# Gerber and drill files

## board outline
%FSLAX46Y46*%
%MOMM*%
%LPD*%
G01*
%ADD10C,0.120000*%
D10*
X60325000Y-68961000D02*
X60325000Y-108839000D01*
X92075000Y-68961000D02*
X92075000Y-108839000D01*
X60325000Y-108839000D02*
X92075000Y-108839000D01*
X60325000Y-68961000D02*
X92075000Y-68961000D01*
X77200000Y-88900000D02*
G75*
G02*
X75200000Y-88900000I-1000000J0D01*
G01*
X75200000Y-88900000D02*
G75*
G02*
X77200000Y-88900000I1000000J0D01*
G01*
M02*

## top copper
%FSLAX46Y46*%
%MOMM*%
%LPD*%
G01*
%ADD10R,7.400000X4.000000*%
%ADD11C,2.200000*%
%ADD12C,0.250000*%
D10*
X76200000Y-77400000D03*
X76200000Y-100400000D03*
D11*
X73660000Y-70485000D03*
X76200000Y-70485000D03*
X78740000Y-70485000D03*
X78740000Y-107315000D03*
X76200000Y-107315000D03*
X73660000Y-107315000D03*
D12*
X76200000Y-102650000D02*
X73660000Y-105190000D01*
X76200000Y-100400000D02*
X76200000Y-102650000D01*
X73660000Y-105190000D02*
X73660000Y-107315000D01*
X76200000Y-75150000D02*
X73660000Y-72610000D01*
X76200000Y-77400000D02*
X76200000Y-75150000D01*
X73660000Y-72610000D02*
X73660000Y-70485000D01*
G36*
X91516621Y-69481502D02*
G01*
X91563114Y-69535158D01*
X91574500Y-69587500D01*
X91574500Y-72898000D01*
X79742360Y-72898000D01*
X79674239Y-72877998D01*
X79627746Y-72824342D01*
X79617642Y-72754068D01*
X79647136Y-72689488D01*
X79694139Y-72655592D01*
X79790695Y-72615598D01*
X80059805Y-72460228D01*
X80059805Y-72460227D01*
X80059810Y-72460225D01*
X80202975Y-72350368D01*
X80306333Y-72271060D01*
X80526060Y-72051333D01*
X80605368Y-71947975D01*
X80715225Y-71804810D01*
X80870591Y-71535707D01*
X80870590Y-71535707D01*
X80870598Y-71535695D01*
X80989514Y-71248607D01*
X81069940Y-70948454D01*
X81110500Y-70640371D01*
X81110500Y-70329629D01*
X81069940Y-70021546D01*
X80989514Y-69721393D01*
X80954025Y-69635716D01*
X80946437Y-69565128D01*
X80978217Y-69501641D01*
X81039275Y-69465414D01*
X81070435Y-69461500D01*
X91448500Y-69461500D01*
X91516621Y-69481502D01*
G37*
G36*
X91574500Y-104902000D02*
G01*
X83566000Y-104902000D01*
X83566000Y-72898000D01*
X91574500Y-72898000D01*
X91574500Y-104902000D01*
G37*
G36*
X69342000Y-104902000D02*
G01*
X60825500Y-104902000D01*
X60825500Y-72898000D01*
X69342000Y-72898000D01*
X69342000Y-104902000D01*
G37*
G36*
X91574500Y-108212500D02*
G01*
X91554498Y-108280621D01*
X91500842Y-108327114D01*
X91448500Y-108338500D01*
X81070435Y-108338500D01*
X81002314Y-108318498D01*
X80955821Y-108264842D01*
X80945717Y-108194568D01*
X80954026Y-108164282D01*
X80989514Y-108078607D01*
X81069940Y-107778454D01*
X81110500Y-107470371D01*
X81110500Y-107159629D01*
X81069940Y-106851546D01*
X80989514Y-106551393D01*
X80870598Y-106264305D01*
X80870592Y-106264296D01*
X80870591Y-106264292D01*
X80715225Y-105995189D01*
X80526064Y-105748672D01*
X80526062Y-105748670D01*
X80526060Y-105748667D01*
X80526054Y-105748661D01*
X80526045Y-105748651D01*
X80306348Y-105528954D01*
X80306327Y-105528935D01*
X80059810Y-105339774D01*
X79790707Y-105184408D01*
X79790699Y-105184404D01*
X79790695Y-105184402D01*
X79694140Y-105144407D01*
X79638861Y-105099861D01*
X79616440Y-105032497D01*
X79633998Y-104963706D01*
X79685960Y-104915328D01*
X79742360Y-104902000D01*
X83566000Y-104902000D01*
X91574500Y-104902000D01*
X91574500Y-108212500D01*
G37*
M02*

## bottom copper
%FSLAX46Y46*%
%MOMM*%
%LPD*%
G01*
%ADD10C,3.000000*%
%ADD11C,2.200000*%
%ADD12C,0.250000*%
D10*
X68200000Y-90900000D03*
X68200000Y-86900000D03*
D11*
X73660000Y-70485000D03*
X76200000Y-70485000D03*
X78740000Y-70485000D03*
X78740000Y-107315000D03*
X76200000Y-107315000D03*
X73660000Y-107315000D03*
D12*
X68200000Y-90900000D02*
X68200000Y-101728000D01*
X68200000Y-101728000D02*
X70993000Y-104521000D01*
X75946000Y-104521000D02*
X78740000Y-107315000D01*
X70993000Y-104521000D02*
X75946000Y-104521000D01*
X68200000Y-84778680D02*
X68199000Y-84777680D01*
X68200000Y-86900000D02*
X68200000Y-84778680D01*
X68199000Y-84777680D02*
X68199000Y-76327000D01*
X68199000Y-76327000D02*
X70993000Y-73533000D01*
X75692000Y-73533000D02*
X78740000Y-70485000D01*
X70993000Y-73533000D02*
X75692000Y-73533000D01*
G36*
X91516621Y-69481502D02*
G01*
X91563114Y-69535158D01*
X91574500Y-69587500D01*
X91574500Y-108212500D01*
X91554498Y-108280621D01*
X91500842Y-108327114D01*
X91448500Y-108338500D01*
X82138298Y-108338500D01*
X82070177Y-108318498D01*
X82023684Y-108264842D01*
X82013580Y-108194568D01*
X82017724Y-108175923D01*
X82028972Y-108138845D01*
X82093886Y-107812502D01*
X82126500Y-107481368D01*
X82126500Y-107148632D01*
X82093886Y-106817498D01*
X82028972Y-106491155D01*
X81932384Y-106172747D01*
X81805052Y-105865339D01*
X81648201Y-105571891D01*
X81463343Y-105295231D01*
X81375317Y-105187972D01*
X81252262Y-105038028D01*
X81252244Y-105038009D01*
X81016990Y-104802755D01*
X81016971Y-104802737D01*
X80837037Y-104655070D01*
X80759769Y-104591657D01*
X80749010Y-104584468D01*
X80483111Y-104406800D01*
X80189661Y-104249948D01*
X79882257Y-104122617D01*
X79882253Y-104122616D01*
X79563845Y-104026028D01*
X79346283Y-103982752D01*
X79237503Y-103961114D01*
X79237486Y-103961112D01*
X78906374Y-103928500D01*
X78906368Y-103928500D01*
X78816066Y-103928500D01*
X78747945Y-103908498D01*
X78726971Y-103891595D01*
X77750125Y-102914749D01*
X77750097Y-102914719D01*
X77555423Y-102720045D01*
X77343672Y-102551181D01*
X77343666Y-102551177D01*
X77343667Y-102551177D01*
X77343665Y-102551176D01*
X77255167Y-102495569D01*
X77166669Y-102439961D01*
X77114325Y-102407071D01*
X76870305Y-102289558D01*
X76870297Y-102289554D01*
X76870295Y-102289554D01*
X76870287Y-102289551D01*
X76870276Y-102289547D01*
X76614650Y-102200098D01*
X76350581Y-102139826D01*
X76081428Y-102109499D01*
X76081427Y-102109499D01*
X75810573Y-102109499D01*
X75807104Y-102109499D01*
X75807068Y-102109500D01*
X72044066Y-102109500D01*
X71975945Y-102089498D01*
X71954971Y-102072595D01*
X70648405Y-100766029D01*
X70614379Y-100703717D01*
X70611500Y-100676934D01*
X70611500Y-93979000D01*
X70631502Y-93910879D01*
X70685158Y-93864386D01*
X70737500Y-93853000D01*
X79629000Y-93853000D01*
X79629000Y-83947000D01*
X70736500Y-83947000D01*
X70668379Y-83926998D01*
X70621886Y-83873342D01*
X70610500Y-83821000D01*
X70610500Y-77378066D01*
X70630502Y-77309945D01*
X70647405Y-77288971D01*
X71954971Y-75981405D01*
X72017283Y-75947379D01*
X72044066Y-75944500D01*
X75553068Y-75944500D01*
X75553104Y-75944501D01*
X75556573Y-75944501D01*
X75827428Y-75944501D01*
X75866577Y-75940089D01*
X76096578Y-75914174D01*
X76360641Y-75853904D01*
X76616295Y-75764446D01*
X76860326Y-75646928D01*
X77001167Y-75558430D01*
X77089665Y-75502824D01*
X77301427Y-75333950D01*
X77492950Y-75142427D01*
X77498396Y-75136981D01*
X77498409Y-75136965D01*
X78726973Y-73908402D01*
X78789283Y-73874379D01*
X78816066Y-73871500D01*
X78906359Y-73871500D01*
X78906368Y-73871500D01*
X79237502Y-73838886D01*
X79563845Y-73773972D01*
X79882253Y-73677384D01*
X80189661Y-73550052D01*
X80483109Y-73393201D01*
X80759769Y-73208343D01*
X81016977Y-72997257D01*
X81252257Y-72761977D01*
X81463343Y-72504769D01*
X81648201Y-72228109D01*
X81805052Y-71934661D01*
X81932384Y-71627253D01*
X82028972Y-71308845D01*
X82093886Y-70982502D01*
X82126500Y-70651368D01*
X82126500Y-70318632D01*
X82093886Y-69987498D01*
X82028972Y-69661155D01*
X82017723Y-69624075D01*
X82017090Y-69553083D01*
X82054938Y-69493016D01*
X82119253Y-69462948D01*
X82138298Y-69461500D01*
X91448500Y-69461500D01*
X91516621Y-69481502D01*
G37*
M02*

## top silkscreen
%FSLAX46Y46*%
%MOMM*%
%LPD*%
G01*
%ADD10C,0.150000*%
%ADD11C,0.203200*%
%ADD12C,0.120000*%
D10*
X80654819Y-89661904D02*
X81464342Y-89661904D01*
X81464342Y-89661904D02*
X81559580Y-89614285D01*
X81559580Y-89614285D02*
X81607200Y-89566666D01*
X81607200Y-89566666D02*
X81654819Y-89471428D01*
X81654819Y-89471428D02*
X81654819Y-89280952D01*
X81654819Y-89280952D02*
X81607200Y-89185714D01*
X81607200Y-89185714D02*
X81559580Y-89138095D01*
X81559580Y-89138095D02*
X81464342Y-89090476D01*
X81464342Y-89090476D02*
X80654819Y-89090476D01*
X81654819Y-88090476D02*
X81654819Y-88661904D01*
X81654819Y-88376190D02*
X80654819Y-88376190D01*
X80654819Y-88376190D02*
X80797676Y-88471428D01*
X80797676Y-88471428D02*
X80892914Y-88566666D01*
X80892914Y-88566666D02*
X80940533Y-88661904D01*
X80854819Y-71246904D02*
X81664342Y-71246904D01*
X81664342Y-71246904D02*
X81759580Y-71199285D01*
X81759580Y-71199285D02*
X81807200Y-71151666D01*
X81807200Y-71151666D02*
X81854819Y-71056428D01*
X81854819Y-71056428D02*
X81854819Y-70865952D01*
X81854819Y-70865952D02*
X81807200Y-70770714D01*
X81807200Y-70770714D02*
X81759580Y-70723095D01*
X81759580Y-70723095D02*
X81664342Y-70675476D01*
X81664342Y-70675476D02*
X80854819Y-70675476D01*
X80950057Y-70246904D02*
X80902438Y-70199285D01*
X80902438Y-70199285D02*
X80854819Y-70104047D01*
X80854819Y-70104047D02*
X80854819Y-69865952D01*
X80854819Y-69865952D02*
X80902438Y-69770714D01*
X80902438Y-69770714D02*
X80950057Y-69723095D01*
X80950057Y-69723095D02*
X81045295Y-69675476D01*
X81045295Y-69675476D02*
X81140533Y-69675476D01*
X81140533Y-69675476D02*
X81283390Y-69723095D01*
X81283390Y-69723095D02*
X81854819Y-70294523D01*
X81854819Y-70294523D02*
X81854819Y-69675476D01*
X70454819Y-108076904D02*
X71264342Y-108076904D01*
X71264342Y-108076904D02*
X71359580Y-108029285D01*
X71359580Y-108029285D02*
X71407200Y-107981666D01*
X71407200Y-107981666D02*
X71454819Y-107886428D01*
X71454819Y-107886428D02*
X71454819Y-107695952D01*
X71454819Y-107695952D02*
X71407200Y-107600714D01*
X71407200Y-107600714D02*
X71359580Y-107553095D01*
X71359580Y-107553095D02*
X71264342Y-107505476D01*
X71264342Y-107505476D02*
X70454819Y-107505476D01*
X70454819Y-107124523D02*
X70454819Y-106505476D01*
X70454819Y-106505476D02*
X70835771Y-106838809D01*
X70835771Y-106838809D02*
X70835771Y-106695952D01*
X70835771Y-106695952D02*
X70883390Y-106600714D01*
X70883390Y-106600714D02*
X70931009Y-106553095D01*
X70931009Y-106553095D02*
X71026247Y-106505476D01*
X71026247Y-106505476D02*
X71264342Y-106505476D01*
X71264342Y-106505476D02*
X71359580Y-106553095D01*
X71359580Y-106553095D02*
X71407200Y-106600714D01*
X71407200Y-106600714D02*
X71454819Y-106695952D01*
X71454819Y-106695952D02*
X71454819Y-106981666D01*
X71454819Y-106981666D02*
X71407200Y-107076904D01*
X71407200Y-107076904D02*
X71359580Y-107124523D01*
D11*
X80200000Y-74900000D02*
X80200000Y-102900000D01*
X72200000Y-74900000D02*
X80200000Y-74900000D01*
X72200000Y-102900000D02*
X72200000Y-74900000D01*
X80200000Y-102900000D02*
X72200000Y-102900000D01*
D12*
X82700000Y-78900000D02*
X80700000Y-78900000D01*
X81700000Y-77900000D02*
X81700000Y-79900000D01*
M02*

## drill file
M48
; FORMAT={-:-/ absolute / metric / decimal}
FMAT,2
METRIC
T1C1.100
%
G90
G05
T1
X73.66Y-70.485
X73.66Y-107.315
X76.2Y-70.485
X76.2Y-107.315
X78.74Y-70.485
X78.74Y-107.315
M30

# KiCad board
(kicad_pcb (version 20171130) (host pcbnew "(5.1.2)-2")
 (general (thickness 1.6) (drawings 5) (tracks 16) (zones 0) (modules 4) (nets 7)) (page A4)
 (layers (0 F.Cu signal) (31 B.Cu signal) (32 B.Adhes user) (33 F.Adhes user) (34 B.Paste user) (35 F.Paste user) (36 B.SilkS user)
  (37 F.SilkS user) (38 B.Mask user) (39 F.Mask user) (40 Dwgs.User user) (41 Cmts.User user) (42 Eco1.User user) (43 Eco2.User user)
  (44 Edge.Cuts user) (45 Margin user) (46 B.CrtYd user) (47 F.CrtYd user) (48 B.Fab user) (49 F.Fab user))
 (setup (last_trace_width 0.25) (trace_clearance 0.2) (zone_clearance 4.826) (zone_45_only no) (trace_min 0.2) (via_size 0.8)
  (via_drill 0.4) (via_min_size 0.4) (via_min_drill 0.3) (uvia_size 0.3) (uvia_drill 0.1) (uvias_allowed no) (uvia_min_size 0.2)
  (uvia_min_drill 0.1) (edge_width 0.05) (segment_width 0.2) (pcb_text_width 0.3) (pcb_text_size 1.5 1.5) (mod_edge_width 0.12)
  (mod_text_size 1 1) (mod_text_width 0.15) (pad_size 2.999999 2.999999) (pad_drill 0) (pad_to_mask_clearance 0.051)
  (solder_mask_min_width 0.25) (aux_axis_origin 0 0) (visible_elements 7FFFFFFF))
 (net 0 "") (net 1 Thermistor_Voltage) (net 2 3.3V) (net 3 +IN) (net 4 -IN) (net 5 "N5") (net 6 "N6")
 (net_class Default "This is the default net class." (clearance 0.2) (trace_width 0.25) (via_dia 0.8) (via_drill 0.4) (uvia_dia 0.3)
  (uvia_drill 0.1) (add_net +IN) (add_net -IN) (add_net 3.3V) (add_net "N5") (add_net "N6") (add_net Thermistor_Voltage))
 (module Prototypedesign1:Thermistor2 (layer B.Cu) (at 76.2 88.9 180)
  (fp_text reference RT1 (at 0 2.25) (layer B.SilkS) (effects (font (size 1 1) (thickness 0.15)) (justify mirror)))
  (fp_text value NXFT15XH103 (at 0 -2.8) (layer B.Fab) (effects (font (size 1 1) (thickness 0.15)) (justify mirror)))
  (pad 2 smd circle (at 8 -2 180) (size 3 3) (layers B.Cu B.Paste B.Mask) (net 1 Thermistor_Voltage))
  (pad 1 smd circle (at 8 2 180) (size 3 3) (layers B.Cu B.Paste B.Mask) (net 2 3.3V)))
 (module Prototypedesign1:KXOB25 (layer F.Cu) (at 76.2 88.9 270)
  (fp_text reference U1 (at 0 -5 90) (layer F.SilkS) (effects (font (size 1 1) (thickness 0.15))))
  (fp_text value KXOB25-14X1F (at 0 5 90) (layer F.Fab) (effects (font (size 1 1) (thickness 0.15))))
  (fp_line (start -14 -4) (end 14 -4) (layer F.SilkS) (width 0.2032))
  (fp_line (start -14 4) (end -14 -4) (layer F.SilkS) (width 0.2032))
  (fp_line (start 14 4) (end -14 4) (layer F.SilkS) (width 0.2032))
  (fp_line (start 14 -4) (end 14 4) (layer F.SilkS) (width 0.2032))
  (fp_line (start -10 -6.5) (end -10 -4.5) (layer F.SilkS) (width 0.12))
  (fp_line (start -11 -5.5) (end -9 -5.5) (layer F.SilkS) (width 0.12))
  (pad 1 smd rect (at -11.5 0 270) (size 4 7.4) (layers F.Cu F.Paste F.Mask) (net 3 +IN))
  (pad 2 smd rect (at 11.5 0 270) (size 4 7.4) (layers F.Cu F.Paste F.Mask) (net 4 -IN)))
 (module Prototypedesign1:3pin (layer F.Cu) (at 76.2 70.485 270)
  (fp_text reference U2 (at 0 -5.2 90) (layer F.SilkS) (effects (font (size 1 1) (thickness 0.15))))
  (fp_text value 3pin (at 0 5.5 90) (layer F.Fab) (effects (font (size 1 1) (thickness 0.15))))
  (pad 3 thru_hole circle (at 0 2.54 270) (size 2.2 2.2) (drill 1.1) (layers *.Cu *.Mask) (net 3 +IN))
  (pad 2 thru_hole circle (at 0 0 270) (size 2.2 2.2) (drill 1.1) (layers *.Cu *.Mask) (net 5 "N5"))
  (pad 1 thru_hole circle (at 0 -2.54 270) (size 2.2 2.2) (drill 1.1) (layers *.Cu *.Mask) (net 2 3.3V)))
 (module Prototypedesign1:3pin (layer F.Cu) (at 76.2 107.315 90)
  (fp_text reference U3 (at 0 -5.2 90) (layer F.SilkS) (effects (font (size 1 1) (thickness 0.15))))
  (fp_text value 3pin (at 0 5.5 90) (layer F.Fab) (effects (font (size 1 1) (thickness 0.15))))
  (pad 3 thru_hole circle (at 0 2.54 90) (size 2.2 2.2) (drill 1.1) (layers *.Cu *.Mask) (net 1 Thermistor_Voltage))
  (pad 2 thru_hole circle (at 0 0 90) (size 2.2 2.2) (drill 1.1) (layers *.Cu *.Mask) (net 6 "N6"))
  (pad 1 thru_hole circle (at 0 -2.54 90) (size 2.2 2.2) (drill 1.1) (layers *.Cu *.Mask) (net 4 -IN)))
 (gr_line (start 60.325 68.961) (end 60.325 108.839) (layer Edge.Cuts) (width 0.12))
 (gr_line (start 92.075 68.961) (end 92.075 108.839) (layer Edge.Cuts) (width 0.12))
 (gr_line (start 60.325 108.839) (end 92.075 108.839) (layer Edge.Cuts) (width 0.12))
 (gr_line (start 60.325 68.961) (end 92.075 68.961) (layer Edge.Cuts) (width 0.12))
 (gr_circle (center 76.2 88.9) (end 77.2 88.9) (layer Edge.Cuts) (width 0.12))
 (segment (start 68.2 90.9) (end 68.2 101.728) (width 0.25) (layer B.Cu) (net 1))
 (segment (start 68.2 101.728) (end 70.993 104.521) (width 0.25) (layer B.Cu) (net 1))
 (segment (start 75.946 104.521) (end 78.74 107.315) (width 0.25) (layer B.Cu) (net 1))
 (segment (start 70.993 104.521) (end 75.946 104.521) (width 0.25) (layer B.Cu) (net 1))
 (segment (start 68.2 84.77868) (end 68.199 84.77768) (width 0.25) (layer B.Cu) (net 2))
 (segment (start 68.2 86.9) (end 68.2 84.77868) (width 0.25) (layer B.Cu) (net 2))
 (segment (start 68.199 84.77768) (end 68.199 76.327) (width 0.25) (layer B.Cu) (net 2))
 (segment (start 68.199 76.327) (end 70.993 73.533) (width 0.25) (layer B.Cu) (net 2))
 (segment (start 75.692 73.533) (end 78.74 70.485) (width 0.25) (layer B.Cu) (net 2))
 (segment (start 70.993 73.533) (end 75.692 73.533) (width 0.25) (layer B.Cu) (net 2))
 (segment (start 76.2 102.65) (end 73.66 105.19) (width 0.25) (layer F.Cu) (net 4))
 (segment (start 76.2 100.4) (end 76.2 102.65) (width 0.25) (layer F.Cu) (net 4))
 (segment (start 73.66 105.19) (end 73.66 107.315) (width 0.25) (layer F.Cu) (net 4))
 (segment (start 76.2 75.15) (end 73.66 72.61) (width 0.25) (layer F.Cu) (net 3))
 (segment (start 76.2 77.4) (end 76.2 75.15) (width 0.25) (layer F.Cu) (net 3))
 (segment (start 73.66 72.61) (end 73.66 70.485) (width 0.25) (layer F.Cu) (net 3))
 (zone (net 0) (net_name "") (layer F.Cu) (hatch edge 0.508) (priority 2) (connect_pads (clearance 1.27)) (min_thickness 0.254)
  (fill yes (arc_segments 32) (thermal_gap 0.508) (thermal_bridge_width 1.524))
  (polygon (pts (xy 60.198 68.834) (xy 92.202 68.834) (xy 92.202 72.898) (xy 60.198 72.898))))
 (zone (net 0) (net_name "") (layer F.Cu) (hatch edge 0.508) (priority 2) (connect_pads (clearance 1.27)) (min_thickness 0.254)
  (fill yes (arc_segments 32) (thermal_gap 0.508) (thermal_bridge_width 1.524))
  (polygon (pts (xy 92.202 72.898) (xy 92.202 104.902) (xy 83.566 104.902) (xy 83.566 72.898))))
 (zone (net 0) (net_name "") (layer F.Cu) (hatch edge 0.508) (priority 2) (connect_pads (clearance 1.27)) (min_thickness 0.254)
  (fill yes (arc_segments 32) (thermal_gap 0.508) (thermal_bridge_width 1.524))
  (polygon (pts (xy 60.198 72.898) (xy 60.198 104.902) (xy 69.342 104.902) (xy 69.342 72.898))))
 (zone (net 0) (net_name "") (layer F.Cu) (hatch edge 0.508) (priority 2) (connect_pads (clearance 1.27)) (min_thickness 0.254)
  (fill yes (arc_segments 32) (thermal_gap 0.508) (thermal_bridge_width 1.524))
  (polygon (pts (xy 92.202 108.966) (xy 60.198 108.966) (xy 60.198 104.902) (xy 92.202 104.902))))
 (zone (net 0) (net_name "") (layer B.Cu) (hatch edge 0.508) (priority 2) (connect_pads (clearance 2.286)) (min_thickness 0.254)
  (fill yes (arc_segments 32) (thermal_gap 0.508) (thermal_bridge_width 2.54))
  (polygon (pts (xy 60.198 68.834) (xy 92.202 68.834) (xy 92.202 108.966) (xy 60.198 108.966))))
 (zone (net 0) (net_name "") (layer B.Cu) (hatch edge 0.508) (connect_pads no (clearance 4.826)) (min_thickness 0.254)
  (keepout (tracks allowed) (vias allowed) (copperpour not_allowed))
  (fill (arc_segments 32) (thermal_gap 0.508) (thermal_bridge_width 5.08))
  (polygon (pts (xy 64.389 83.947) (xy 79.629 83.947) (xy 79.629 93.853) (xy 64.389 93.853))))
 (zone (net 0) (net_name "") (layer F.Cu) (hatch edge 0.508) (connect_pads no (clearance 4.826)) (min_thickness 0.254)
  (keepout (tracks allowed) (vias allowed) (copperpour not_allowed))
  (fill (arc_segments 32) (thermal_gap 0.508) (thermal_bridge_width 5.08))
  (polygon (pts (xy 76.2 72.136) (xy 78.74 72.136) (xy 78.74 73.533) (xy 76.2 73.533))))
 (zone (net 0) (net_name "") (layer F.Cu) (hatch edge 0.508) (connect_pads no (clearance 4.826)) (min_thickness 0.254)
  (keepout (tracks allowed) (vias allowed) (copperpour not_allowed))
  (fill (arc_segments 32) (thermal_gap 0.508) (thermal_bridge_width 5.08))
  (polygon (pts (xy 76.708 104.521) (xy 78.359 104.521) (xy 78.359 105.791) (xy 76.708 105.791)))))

